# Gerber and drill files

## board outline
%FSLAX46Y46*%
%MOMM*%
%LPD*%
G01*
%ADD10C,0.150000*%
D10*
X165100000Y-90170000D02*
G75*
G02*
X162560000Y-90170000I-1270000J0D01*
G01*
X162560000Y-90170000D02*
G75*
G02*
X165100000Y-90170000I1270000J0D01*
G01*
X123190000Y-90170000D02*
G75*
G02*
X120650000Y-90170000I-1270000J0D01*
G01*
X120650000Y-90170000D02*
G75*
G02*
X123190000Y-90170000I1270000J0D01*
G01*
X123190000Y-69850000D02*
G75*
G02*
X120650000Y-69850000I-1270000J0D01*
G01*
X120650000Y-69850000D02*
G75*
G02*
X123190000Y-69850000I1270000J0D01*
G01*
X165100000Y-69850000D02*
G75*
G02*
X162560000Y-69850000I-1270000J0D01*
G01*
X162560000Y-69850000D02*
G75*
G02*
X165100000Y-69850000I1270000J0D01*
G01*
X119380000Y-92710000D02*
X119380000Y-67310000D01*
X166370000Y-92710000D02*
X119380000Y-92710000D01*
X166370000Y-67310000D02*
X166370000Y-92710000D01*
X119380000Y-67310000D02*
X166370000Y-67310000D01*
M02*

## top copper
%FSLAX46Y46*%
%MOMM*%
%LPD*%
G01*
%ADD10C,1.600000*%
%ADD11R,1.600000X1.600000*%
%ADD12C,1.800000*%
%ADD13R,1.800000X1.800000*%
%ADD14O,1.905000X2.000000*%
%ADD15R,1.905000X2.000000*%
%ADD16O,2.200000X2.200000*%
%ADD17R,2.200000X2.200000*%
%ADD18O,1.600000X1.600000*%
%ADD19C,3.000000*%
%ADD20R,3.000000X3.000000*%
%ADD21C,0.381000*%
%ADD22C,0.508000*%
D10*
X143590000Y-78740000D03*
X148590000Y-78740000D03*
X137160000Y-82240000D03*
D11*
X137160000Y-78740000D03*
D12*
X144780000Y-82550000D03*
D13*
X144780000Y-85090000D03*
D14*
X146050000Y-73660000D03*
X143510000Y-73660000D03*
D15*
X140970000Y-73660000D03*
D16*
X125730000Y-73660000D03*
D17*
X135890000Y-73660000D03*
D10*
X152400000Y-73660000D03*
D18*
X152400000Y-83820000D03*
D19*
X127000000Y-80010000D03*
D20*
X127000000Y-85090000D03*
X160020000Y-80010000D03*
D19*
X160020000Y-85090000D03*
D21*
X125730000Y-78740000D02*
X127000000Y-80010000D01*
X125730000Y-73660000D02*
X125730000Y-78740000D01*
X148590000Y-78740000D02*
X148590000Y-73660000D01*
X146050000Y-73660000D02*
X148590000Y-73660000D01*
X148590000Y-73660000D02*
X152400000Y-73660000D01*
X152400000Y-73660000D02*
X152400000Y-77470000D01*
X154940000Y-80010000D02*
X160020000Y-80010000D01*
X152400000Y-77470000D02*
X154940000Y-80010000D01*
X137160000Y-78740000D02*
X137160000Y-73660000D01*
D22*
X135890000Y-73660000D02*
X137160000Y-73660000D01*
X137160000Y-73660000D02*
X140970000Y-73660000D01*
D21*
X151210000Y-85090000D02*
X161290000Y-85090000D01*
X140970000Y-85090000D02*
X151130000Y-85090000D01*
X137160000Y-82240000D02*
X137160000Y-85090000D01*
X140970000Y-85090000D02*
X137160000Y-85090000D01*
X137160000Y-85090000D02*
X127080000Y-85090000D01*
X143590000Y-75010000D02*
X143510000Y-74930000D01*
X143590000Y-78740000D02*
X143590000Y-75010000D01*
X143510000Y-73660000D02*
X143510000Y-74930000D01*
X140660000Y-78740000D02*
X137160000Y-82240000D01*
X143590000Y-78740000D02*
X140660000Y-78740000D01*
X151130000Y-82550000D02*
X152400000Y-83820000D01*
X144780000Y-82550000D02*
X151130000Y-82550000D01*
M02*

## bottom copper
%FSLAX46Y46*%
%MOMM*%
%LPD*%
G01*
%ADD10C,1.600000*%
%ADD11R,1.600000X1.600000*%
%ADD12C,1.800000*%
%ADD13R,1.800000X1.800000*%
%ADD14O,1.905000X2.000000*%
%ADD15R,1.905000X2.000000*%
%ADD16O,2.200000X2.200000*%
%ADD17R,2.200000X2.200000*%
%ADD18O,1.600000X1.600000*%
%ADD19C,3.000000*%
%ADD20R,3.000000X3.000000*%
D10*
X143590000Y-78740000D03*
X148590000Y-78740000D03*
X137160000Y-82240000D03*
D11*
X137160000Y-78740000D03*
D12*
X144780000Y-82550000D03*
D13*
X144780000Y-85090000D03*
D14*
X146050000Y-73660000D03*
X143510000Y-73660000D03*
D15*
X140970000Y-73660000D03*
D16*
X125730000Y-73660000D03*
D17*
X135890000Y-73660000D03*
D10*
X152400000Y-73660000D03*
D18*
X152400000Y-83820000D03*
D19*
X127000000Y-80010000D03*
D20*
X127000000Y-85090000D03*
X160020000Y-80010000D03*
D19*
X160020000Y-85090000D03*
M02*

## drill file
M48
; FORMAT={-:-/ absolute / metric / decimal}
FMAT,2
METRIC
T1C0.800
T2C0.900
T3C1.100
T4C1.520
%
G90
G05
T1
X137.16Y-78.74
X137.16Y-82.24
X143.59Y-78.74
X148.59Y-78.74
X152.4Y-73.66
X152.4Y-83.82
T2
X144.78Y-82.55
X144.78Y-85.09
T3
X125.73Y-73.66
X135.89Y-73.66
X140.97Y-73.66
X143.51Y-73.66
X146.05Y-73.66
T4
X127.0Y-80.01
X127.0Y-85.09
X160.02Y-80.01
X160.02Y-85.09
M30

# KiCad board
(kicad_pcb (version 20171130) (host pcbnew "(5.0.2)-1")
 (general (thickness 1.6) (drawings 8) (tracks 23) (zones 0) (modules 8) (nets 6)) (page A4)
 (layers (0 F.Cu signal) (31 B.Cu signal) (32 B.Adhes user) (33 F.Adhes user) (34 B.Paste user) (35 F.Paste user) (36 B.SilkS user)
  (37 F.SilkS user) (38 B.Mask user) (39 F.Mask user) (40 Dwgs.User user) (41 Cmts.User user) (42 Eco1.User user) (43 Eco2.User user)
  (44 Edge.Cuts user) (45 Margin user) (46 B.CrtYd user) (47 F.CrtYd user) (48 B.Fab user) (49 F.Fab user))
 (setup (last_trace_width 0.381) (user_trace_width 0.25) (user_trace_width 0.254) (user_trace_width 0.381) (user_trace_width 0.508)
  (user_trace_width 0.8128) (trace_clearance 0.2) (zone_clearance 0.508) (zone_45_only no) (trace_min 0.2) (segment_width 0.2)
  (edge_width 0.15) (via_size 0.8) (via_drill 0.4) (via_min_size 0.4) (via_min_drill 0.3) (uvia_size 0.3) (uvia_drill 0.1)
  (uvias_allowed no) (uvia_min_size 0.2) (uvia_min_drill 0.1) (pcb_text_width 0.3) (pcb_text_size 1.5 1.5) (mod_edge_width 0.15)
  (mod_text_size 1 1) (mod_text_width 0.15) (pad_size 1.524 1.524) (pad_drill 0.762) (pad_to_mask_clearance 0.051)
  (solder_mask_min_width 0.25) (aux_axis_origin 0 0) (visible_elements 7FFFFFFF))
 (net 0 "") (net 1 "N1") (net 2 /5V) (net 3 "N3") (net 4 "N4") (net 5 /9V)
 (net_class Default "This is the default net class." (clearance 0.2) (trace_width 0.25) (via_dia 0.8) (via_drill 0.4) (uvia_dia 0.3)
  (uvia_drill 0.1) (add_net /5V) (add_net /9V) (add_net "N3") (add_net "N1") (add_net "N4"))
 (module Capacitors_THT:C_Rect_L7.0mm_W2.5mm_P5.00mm (layer F.Cu) (at 148.59 78.74 180)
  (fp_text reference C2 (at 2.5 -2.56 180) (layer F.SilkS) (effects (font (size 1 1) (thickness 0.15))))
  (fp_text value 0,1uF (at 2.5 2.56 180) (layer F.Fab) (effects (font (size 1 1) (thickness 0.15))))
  (pad 2 thru_hole circle (at 5 0 180) (size 1.6 1.6) (drill 0.8) (layers *.Cu *.Mask) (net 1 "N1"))
  (pad 1 thru_hole circle (at 0 0 180) (size 1.6 1.6) (drill 0.8) (layers *.Cu *.Mask) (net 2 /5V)))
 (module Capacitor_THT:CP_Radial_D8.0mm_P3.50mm (layer F.Cu) (at 137.16 78.74 270)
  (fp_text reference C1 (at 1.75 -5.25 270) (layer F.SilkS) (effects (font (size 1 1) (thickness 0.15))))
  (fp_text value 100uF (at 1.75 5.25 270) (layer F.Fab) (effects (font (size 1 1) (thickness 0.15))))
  (pad 2 thru_hole circle (at 3.5 0 270) (size 1.6 1.6) (drill 0.8) (layers *.Cu *.Mask) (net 1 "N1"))
  (pad 1 thru_hole rect (at 0 0 270) (size 1.6 1.6) (drill 0.8) (layers *.Cu *.Mask) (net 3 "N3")))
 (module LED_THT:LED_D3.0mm (layer F.Cu) (at 144.78 85.09 90)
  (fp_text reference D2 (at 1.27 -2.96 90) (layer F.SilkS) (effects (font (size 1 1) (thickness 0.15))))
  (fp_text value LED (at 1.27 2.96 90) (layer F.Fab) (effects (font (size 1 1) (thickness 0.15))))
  (pad 2 thru_hole circle (at 2.54 0 90) (size 1.8 1.8) (drill 0.9) (layers *.Cu *.Mask) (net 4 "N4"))
  (pad 1 thru_hole rect (at 0 0 90) (size 1.8 1.8) (drill 0.9) (layers *.Cu *.Mask) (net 1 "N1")))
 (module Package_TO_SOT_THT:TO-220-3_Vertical (layer F.Cu) (at 140.97 73.66)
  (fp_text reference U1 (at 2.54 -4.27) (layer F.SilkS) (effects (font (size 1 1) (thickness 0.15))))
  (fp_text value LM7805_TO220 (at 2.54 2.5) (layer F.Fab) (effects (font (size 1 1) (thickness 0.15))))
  (pad 3 thru_hole oval (at 5.08 0) (size 1.905 2) (drill 1.1) (layers *.Cu *.Mask) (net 2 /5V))
  (pad 2 thru_hole oval (at 2.54 0) (size 1.905 2) (drill 1.1) (layers *.Cu *.Mask) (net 1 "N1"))
  (pad 1 thru_hole rect (at 0 0) (size 1.905 2) (drill 1.1) (layers *.Cu *.Mask) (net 3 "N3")))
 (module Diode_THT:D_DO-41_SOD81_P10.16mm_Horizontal (layer F.Cu) (at 135.89 73.66 180)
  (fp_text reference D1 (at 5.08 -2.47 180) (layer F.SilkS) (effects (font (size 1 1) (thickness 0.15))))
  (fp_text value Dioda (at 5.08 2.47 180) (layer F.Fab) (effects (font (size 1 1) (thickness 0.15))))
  (pad 2 thru_hole oval (at 10.16 0 180) (size 2.2 2.2) (drill 1.1) (layers *.Cu *.Mask) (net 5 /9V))
  (pad 1 thru_hole rect (at 0 0 180) (size 2.2 2.2) (drill 1.1) (layers *.Cu *.Mask) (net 3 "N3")))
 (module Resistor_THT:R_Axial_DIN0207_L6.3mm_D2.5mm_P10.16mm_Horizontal (layer F.Cu) (at 152.4 73.66 270)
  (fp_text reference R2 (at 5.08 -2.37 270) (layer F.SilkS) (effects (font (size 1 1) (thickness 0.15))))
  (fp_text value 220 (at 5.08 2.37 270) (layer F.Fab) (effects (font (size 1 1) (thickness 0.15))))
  (pad 1 thru_hole circle (at 0 0 270) (size 1.6 1.6) (drill 0.8) (layers *.Cu *.Mask) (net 2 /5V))
  (pad 2 thru_hole oval (at 10.16 0 270) (size 1.6 1.6) (drill 0.8) (layers *.Cu *.Mask) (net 4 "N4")))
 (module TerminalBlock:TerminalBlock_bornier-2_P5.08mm (layer F.Cu) (at 127 85.09 90)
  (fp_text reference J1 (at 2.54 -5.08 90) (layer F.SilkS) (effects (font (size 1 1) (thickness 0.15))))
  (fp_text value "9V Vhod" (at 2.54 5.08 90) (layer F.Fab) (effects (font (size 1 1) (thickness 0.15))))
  (pad 2 thru_hole circle (at 5.08 0 90) (size 3 3) (drill 1.52) (layers *.Cu *.Mask) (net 5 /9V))
  (pad 1 thru_hole rect (at 0 0 90) (size 3 3) (drill 1.52) (layers *.Cu *.Mask) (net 1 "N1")))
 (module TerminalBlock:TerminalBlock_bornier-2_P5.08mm (layer F.Cu) (at 160.02 80.01 270)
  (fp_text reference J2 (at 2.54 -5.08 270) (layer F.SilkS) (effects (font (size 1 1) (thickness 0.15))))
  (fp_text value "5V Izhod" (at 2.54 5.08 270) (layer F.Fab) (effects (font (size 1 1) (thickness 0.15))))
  (pad 1 thru_hole rect (at 0 0 270) (size 3 3) (drill 1.52) (layers *.Cu *.Mask) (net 2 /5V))
  (pad 2 thru_hole circle (at 5.08 0 270) (size 3 3) (drill 1.52) (layers *.Cu *.Mask) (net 1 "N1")))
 (gr_circle (center 163.83 90.17) (end 163.83 91.44) (layer Edge.Cuts) (width 0.15))
 (gr_circle (center 121.92 90.17) (end 121.92 91.44) (layer Edge.Cuts) (width 0.15))
 (gr_circle (center 121.92 69.85) (end 120.65 69.85) (layer Edge.Cuts) (width 0.15))
 (gr_circle (center 163.83 69.85) (end 163.83 68.58) (layer Edge.Cuts) (width 0.15))
 (gr_line (start 119.38 92.71) (end 119.38 67.31) (layer Edge.Cuts) (width 0.15))
 (gr_line (start 166.37 92.71) (end 119.38 92.71) (layer Edge.Cuts) (width 0.15))
 (gr_line (start 166.37 67.31) (end 166.37 92.71) (layer Edge.Cuts) (width 0.15))
 (gr_line (start 119.38 67.31) (end 166.37 67.31) (layer Edge.Cuts) (width 0.15))
 (segment (start 125.73 78.74) (end 127 80.01) (width 0.381) (layer F.Cu) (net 5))
 (segment (start 125.73 73.66) (end 125.73 78.74) (width 0.381) (layer F.Cu) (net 5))
 (segment (start 148.59 78.74) (end 148.59 73.66) (width 0.381) (layer F.Cu) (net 2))
 (segment (start 146.05 73.66) (end 148.59 73.66) (width 0.381) (layer F.Cu) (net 2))
 (segment (start 148.59 73.66) (end 152.4 73.66) (width 0.381) (layer F.Cu) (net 2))
 (segment (start 152.4 73.66) (end 152.4 77.47) (width 0.381) (layer F.Cu) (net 2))
 (segment (start 154.94 80.01) (end 160.02 80.01) (width 0.381) (layer F.Cu) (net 2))
 (segment (start 152.4 77.47) (end 154.94 80.01) (width 0.381) (layer F.Cu) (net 2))
 (segment (start 137.16 78.74) (end 137.16 73.66) (width 0.381) (layer F.Cu) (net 3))
 (segment (start 135.89 73.66) (end 137.16 73.66) (width 0.508) (layer F.Cu) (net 3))
 (segment (start 137.16 73.66) (end 140.97 73.66) (width 0.508) (layer F.Cu) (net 3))
 (segment (start 151.21 85.09) (end 161.29 85.09) (width 0.381) (layer F.Cu) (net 1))
 (segment (start 140.97 85.09) (end 151.13 85.09) (width 0.381) (layer F.Cu) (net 1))
 (segment (start 137.16 82.24) (end 137.16 85.09) (width 0.381) (layer F.Cu) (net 1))
 (segment (start 140.97 85.09) (end 137.16 85.09) (width 0.381) (layer F.Cu) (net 1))
 (segment (start 137.16 85.09) (end 127.08 85.09) (width 0.381) (layer F.Cu) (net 1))
 (segment (start 143.59 75.01) (end 143.51 74.93) (width 0.381) (layer F.Cu) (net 1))
 (segment (start 143.59 78.74) (end 143.59 75.01) (width 0.381) (layer F.Cu) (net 1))
 (segment (start 143.51 73.66) (end 143.51 74.93) (width 0.381) (layer F.Cu) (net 1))
 (segment (start 140.66 78.74) (end 137.16 82.24) (width 0.381) (layer F.Cu) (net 1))
 (segment (start 143.59 78.74) (end 140.66 78.74) (width 0.381) (layer F.Cu) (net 1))
 (segment (start 151.13 82.55) (end 152.4 83.82) (width 0.381) (layer F.Cu) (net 4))
 (segment (start 144.78 82.55) (end 151.13 82.55) (width 0.381) (layer F.Cu) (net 4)))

